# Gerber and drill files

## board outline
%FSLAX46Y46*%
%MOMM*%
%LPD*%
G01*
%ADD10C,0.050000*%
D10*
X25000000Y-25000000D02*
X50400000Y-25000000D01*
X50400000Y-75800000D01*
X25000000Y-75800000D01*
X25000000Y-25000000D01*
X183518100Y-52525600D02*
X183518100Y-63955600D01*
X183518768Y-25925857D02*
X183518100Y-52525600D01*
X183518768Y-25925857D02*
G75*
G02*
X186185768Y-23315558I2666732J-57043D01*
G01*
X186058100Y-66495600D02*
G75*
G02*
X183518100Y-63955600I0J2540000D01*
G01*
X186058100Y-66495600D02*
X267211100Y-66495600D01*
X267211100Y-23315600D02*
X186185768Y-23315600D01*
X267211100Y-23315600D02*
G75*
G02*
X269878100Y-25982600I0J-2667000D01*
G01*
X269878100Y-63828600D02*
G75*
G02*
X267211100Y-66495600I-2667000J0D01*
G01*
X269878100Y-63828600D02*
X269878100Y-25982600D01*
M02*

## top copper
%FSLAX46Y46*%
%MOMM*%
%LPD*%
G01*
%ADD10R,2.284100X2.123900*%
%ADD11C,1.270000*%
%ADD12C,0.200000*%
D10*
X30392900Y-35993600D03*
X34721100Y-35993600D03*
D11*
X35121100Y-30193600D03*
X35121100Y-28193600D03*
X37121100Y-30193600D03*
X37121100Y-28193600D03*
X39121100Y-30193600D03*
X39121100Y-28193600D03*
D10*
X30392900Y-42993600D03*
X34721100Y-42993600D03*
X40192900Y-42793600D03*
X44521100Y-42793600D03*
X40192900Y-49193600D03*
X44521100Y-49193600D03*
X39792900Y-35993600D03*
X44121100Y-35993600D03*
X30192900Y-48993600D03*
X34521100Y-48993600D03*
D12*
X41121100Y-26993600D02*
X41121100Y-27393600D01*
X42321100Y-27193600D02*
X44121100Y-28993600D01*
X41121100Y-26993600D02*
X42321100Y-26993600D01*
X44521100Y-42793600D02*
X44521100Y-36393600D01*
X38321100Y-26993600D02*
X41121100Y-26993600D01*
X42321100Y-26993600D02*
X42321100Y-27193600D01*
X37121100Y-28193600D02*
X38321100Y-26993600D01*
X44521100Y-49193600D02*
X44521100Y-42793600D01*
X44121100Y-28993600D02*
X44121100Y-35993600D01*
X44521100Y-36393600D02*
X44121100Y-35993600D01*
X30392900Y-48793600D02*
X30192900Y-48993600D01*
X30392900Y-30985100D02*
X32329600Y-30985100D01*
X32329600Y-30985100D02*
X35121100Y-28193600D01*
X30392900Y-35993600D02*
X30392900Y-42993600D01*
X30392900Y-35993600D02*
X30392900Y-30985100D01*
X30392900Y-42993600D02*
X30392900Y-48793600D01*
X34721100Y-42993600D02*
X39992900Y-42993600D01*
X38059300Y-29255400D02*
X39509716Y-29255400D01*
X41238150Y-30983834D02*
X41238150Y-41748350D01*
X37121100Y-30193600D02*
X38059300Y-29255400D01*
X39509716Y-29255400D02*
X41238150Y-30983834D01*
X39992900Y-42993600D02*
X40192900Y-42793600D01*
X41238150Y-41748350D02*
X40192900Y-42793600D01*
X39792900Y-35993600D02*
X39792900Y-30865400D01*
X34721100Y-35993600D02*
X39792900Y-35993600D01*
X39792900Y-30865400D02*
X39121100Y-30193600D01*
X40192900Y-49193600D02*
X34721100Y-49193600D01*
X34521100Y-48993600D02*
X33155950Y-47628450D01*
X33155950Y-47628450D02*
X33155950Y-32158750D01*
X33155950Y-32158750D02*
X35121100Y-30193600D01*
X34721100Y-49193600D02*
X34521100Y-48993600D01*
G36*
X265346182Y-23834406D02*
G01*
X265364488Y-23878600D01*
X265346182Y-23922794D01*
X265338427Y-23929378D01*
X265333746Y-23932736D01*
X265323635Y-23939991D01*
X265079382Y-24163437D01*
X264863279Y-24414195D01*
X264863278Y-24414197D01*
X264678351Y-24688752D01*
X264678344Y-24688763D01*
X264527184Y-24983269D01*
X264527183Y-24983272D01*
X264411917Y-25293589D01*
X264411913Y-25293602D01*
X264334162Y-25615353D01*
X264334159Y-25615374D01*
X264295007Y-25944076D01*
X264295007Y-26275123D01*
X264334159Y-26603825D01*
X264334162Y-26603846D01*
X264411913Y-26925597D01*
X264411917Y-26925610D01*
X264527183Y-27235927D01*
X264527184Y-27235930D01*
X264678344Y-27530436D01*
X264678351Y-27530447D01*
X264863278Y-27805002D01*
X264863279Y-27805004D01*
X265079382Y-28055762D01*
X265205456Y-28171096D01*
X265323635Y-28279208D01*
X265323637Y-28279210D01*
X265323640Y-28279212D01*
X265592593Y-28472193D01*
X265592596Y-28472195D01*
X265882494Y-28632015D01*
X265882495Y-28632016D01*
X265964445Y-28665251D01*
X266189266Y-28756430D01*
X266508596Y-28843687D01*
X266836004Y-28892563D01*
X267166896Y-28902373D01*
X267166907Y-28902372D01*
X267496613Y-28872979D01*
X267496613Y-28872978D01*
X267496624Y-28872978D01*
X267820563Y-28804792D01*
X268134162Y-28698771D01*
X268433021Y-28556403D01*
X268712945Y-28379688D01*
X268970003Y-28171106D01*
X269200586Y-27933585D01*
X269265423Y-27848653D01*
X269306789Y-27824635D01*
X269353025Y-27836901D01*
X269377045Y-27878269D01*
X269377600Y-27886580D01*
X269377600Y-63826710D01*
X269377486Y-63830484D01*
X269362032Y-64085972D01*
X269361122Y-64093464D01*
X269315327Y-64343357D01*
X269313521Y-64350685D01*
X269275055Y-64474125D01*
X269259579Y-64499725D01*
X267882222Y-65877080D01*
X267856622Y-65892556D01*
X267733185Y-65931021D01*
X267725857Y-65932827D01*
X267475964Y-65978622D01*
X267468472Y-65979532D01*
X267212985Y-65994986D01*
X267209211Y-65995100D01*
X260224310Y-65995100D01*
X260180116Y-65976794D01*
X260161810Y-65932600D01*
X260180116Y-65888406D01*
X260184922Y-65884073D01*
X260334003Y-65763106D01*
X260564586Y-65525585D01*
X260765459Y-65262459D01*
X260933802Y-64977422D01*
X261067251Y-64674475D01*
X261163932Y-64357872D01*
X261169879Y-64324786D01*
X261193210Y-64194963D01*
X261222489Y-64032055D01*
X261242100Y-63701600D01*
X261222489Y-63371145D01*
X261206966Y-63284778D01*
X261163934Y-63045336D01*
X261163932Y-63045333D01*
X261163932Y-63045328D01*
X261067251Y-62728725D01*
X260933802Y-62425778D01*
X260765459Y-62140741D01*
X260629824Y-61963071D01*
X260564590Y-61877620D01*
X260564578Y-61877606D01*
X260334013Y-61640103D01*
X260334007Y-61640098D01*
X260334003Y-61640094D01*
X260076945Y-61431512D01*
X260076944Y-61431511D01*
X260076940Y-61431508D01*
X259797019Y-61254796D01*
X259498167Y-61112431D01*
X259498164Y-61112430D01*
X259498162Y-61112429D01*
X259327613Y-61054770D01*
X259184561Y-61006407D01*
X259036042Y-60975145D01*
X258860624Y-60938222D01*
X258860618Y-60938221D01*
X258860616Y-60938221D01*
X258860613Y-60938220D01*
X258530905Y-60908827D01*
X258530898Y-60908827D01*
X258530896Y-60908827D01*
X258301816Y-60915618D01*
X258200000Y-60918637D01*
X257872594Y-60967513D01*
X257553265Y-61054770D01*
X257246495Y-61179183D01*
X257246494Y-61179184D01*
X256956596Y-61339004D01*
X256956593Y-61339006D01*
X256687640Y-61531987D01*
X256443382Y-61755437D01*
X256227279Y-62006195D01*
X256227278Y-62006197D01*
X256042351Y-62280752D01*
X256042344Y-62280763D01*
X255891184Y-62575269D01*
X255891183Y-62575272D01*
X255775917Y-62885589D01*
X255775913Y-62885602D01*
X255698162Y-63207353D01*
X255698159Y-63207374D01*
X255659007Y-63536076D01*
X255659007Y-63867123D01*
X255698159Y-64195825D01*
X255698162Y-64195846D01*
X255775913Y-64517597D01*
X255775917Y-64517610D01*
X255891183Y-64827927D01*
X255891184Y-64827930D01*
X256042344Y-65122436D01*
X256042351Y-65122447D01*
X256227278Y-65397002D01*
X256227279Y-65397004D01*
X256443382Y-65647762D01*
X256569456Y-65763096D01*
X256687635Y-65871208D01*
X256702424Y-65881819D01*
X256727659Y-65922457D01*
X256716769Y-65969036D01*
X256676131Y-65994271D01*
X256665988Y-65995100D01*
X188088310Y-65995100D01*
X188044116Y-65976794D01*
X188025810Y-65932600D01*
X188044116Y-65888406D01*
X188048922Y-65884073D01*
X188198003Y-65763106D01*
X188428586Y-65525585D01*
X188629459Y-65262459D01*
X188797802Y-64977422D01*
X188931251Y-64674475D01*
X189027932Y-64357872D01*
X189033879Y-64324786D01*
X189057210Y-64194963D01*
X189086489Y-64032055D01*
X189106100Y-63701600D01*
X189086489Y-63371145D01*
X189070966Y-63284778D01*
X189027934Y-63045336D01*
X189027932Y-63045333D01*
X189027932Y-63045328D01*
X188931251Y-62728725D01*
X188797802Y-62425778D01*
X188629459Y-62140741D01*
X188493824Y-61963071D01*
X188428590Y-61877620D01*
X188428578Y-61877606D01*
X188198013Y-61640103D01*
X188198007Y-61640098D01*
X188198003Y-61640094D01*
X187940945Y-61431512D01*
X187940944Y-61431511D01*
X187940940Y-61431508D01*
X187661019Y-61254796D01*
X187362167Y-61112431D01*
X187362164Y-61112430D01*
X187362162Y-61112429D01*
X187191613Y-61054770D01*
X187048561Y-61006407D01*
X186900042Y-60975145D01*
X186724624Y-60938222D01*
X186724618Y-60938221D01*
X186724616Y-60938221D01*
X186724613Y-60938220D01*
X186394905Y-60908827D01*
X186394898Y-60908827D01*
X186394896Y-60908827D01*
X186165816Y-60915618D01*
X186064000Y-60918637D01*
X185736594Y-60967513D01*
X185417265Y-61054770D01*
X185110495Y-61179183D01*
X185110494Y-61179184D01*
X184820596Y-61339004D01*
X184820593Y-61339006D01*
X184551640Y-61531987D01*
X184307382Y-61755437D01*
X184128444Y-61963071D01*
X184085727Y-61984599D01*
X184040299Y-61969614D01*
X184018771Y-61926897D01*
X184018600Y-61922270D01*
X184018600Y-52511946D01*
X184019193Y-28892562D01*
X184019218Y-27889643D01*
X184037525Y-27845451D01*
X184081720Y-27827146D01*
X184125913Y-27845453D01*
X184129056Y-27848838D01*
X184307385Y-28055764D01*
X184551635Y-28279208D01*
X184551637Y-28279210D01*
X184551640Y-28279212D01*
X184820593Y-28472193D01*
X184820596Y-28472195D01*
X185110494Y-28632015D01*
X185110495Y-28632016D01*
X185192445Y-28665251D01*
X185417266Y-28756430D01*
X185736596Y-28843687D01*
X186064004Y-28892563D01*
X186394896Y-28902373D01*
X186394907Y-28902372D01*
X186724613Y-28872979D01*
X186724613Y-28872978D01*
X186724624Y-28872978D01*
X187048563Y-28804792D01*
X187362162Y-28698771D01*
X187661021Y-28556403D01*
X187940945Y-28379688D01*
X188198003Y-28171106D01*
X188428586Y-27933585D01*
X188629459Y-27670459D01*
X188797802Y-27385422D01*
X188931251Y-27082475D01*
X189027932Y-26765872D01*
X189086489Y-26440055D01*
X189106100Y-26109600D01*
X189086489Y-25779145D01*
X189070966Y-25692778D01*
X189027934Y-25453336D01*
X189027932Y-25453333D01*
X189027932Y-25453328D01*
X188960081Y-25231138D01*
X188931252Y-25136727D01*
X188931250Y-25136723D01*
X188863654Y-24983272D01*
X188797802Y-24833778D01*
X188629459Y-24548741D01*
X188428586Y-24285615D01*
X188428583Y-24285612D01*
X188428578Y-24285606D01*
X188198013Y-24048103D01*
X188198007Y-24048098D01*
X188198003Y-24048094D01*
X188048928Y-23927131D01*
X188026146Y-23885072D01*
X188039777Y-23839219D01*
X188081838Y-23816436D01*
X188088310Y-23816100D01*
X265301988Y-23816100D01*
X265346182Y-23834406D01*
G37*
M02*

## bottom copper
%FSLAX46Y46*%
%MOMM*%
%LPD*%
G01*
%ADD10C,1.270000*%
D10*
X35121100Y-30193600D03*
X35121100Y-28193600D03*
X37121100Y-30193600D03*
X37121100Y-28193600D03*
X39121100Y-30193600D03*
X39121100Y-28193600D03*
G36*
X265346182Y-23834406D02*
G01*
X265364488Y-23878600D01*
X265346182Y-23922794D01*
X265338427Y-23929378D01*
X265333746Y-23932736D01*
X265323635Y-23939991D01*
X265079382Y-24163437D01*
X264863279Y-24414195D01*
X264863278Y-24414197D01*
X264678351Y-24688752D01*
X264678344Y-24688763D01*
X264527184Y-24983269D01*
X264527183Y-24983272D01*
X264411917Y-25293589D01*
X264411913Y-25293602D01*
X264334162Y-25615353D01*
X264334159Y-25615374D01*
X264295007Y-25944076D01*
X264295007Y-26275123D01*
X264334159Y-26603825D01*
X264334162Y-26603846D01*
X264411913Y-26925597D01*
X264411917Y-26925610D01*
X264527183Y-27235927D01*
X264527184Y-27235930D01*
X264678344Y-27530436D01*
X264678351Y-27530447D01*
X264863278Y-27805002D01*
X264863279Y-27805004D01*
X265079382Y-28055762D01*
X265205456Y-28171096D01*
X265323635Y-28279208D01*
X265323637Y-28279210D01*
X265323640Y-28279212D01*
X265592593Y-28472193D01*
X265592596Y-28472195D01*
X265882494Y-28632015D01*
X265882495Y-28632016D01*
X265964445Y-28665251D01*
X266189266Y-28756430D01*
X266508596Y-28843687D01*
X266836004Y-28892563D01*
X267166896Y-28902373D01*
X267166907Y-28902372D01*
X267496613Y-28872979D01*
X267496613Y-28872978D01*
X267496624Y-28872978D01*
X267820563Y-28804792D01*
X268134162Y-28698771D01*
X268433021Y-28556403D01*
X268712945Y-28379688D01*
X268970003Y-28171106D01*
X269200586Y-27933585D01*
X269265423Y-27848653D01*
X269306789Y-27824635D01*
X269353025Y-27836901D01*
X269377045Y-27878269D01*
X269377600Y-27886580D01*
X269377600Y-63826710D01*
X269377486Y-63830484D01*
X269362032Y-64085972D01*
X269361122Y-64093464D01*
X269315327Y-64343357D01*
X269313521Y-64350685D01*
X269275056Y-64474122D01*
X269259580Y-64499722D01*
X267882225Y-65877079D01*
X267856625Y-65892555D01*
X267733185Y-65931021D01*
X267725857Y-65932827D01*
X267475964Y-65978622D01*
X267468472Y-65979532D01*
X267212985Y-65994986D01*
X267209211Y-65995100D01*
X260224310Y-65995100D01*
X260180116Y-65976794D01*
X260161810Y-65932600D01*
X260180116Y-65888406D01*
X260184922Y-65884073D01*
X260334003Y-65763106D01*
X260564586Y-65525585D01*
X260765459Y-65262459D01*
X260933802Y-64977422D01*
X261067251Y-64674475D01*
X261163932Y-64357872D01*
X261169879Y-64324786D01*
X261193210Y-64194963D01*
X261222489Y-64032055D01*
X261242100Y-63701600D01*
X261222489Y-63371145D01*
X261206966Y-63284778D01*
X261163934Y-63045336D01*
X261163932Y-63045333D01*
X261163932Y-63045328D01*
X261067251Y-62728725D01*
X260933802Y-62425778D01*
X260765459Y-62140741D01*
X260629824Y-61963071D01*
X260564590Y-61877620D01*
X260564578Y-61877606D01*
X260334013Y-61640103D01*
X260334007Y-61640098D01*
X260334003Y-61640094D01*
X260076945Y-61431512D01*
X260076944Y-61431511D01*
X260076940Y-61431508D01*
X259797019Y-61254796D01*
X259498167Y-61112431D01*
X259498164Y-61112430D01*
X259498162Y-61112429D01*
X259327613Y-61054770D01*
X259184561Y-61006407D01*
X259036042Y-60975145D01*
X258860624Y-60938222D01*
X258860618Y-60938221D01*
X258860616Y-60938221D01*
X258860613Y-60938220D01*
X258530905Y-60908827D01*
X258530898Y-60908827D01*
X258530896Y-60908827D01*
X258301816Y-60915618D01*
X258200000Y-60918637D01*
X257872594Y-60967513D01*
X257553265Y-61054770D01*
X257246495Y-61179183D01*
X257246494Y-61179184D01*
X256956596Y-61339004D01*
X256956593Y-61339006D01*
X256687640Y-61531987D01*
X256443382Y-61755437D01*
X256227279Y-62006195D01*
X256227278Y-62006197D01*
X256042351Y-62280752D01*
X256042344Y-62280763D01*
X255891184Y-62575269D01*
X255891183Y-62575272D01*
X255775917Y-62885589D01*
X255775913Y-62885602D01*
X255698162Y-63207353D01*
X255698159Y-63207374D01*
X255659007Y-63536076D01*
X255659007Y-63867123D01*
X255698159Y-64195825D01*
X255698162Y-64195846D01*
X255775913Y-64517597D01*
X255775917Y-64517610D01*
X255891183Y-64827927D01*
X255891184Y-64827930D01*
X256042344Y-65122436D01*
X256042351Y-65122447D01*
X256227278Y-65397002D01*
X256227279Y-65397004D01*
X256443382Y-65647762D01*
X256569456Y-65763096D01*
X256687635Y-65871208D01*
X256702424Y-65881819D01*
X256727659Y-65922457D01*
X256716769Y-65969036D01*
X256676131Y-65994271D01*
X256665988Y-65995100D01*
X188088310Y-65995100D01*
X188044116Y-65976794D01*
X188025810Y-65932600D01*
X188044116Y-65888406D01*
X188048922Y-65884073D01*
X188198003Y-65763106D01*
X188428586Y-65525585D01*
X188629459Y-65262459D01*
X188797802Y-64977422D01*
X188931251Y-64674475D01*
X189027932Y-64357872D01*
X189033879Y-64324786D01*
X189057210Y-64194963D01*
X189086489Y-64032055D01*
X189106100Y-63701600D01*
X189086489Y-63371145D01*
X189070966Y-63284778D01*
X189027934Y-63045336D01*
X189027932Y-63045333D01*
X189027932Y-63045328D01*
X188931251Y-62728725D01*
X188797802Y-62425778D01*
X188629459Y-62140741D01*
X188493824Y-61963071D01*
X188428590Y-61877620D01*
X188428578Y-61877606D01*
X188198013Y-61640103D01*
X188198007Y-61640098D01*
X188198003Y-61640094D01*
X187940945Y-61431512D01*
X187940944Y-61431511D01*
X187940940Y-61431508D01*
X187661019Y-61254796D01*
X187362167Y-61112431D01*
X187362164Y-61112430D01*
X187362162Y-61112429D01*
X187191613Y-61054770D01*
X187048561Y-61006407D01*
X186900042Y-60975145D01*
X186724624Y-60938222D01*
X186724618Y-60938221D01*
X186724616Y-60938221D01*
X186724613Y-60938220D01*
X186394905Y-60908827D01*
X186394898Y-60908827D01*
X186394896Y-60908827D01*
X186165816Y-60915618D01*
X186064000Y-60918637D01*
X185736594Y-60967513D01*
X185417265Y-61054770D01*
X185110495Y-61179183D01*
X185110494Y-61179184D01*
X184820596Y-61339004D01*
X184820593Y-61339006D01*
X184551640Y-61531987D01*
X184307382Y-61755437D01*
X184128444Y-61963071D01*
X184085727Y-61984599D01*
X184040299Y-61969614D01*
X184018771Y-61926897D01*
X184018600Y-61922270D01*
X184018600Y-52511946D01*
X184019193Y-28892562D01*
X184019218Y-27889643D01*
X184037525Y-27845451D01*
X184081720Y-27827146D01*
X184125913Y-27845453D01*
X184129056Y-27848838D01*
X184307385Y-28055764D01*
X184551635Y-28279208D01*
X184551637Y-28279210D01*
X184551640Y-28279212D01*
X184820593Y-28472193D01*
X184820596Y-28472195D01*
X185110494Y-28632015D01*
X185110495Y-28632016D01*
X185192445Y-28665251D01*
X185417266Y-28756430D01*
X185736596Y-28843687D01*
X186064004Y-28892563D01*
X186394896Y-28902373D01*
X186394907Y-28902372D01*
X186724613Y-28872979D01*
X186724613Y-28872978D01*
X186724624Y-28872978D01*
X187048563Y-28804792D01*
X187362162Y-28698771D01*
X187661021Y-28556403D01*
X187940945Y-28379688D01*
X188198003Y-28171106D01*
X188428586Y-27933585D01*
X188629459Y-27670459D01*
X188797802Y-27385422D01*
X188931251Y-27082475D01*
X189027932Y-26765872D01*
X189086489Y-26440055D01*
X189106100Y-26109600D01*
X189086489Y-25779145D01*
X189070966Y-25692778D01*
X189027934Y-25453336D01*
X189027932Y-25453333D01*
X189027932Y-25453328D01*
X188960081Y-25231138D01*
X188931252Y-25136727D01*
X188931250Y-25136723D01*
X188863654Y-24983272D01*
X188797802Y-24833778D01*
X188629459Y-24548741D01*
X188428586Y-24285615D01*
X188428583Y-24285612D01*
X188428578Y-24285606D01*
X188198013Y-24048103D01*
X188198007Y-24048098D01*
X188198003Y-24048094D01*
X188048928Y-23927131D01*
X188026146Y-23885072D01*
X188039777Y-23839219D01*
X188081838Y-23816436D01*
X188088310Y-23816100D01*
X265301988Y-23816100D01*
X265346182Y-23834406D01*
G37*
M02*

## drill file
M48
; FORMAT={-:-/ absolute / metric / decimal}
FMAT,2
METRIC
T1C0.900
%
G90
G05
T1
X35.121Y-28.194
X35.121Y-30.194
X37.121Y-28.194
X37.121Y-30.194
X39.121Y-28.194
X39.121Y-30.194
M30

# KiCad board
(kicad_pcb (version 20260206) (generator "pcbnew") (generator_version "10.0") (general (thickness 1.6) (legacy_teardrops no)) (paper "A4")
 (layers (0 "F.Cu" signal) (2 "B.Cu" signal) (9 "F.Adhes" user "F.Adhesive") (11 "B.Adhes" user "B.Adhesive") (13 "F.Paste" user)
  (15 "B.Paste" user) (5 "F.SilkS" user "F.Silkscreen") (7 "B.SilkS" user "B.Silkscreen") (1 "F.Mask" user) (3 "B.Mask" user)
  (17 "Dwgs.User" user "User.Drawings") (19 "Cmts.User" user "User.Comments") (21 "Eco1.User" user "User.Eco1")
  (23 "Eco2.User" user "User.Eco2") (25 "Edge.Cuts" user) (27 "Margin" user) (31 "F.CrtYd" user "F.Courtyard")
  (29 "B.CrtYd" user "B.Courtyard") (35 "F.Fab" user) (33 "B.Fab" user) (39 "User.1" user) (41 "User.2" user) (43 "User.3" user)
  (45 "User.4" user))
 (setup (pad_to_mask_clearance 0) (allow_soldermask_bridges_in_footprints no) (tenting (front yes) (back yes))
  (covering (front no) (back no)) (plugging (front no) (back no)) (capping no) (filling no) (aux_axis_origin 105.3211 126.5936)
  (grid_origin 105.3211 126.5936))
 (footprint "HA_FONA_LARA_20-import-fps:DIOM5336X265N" (layer "F.Cu") (at 32.557 35.9936)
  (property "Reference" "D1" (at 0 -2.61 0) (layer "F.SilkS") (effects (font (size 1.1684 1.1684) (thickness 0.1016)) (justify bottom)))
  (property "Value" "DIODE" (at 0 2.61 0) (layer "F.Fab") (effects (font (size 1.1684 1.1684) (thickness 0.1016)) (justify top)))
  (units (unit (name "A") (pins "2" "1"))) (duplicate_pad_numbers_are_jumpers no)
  (pad "1" smd rect (at -2.1641 0) (size 2.2841 2.1239) (layers "F.Cu" "F.Mask" "F.Paste") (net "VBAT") (solder_mask_margin 0.0508)
   (solder_paste_margin 0) (thermal_bridge_angle 0))
  (pad "2" smd rect (at 2.1641 0) (size 2.2841 2.1239) (layers "F.Cu" "F.Mask" "F.Paste") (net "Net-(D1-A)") (solder_mask_margin 0.0508)
   (solder_paste_margin 0) (thermal_bridge_angle 0)))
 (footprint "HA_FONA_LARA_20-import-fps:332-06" (layer "F.Cu") (at 37.1211 29.1936)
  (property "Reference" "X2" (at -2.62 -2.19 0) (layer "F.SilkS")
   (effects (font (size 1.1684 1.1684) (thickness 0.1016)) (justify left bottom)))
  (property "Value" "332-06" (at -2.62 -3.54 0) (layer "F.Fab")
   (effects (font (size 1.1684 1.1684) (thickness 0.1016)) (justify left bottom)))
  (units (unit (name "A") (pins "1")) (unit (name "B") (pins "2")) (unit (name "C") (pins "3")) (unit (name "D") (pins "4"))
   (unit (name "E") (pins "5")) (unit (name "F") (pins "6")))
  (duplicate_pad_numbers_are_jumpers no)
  (pad "1" thru_hole circle (at -2 1) (size 1.27 1.27) (drill 0.9) (layers "*.Cu" "*.Mask") (remove_unused_layers no) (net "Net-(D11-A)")
   (solder_mask_margin 0.0508) (thermal_bridge_angle 0))
  (pad "2" thru_hole circle (at -2 -1) (size 1.27 1.27) (drill 0.9) (layers "*.Cu" "*.Mask") (remove_unused_layers no) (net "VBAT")
   (solder_mask_margin 0.0508) (thermal_bridge_angle 0))
  (pad "3" thru_hole circle (at 0 1) (size 1.27 1.27) (drill 0.9) (layers "*.Cu" "*.Mask") (remove_unused_layers no) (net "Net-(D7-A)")
   (solder_mask_margin 0.0508) (thermal_bridge_angle 0))
  (pad "4" thru_hole circle (at 0 -1) (size 1.27 1.27) (drill 0.9) (layers "*.Cu" "*.Mask") (remove_unused_layers no) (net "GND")
   (solder_mask_margin 0.0508) (thermal_bridge_angle 0))
  (pad "5" thru_hole circle (at 2 1) (size 1.27 1.27) (drill 0.9) (layers "*.Cu" "*.Mask") (remove_unused_layers no) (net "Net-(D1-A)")
   (solder_mask_margin 0.0508) (thermal_bridge_angle 0))
  (pad "6" thru_hole circle (at 2 -1) (size 1.27 1.27) (drill 0.9) (layers "*.Cu" "*.Mask") (remove_unused_layers no)
   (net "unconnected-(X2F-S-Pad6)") (solder_mask_margin 0.0508) (thermal_bridge_angle 0)))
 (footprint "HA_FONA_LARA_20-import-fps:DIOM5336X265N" (layer "F.Cu") (at 32.557 42.9936)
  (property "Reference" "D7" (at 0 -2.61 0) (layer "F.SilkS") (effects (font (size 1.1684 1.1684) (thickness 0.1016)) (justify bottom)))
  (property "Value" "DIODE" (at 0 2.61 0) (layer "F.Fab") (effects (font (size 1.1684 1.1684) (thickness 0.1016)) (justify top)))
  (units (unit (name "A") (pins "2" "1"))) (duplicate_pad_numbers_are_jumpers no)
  (pad "1" smd rect (at -2.1641 0) (size 2.2841 2.1239) (layers "F.Cu" "F.Mask" "F.Paste") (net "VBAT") (solder_mask_margin 0.0508)
   (solder_paste_margin 0) (thermal_bridge_angle 0))
  (pad "2" smd rect (at 2.1641 0) (size 2.2841 2.1239) (layers "F.Cu" "F.Mask" "F.Paste") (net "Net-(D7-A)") (solder_mask_margin 0.0508)
   (solder_paste_margin 0) (thermal_bridge_angle 0)))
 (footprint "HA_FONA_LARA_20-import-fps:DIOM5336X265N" (layer "F.Cu") (at 42.357 42.7936)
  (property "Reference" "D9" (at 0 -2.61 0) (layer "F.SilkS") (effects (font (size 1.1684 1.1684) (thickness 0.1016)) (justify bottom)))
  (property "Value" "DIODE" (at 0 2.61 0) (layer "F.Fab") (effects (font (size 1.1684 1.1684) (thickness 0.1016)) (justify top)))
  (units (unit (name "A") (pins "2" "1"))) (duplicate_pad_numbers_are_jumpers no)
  (pad "1" smd rect (at -2.1641 0) (size 2.2841 2.1239) (layers "F.Cu" "F.Mask" "F.Paste") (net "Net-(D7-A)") (solder_mask_margin 0.0508)
   (solder_paste_margin 0) (thermal_bridge_angle 0))
  (pad "2" smd rect (at 2.1641 0) (size 2.2841 2.1239) (layers "F.Cu" "F.Mask" "F.Paste") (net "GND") (solder_mask_margin 0.0508)
   (solder_paste_margin 0) (thermal_bridge_angle 0)))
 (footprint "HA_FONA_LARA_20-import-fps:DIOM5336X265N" (layer "F.Cu") (at 42.357 49.1936)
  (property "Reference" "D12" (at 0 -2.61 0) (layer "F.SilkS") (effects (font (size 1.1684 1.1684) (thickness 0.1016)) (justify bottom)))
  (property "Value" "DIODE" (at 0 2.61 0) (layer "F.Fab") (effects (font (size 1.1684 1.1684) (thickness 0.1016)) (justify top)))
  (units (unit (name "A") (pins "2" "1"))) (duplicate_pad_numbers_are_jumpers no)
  (pad "1" smd rect (at -2.1641 0) (size 2.2841 2.1239) (layers "F.Cu" "F.Mask" "F.Paste") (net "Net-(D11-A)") (solder_mask_margin 0.0508)
   (solder_paste_margin 0) (thermal_bridge_angle 0))
  (pad "2" smd rect (at 2.1641 0) (size 2.2841 2.1239) (layers "F.Cu" "F.Mask" "F.Paste") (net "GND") (solder_mask_margin 0.0508)
   (solder_paste_margin 0) (thermal_bridge_angle 0)))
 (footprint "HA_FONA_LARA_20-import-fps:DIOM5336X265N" (layer "F.Cu") (at 41.957 35.9936)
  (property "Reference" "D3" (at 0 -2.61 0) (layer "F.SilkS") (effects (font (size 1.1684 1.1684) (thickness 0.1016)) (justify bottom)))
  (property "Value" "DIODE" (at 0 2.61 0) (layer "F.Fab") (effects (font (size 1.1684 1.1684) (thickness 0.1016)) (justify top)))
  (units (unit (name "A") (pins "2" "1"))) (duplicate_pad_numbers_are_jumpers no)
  (pad "1" smd rect (at -2.1641 0) (size 2.2841 2.1239) (layers "F.Cu" "F.Mask" "F.Paste") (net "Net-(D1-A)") (solder_mask_margin 0.0508)
   (solder_paste_margin 0) (thermal_bridge_angle 0))
  (pad "2" smd rect (at 2.1641 0) (size 2.2841 2.1239) (layers "F.Cu" "F.Mask" "F.Paste") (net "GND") (solder_mask_margin 0.0508)
   (solder_paste_margin 0) (thermal_bridge_angle 0)))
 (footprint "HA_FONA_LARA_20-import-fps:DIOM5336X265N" (layer "F.Cu") (at 32.357 48.9936)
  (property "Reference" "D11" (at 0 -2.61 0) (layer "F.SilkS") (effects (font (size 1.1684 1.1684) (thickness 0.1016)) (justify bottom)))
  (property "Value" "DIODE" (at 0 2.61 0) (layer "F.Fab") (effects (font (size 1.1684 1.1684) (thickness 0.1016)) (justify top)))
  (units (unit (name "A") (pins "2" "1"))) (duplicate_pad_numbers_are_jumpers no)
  (pad "1" smd rect (at -2.1641 0) (size 2.2841 2.1239) (layers "F.Cu" "F.Mask" "F.Paste") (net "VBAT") (solder_mask_margin 0.0508)
   (solder_paste_margin 0) (thermal_bridge_angle 0))
  (pad "2" smd rect (at 2.1641 0) (size 2.2841 2.1239) (layers "F.Cu" "F.Mask" "F.Paste") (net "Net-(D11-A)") (solder_mask_margin 0.0508)
   (solder_paste_margin 0) (thermal_bridge_angle 0)))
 (gr_rect (start 25 25) (end 50.4 75.8) (stroke (width 0.05) (type solid)) (fill no) (layer "Edge.Cuts"))
 (gr_line (start 183.5181 52.5256) (end 183.5181 63.9556) (stroke (width 0.05) (type solid)) (layer "Edge.Cuts"))
 (gr_line (start 183.518768 25.925857) (end 183.5181 52.5256) (stroke (width 0.05) (type solid)) (layer "Edge.Cuts"))
 (gr_arc (start 183.518768 25.925857) (mid 184.31978 24.076665) (end 186.185768 23.3156) (stroke (width 0.05) (type solid))
  (layer "Edge.Cuts"))
 (gr_arc (start 186.0581 66.4956) (mid 184.262049 65.751651) (end 183.5181 63.9556) (stroke (width 0.05) (type solid)) (layer "Edge.Cuts"))
 (gr_line (start 186.0581 66.4956) (end 267.2111 66.4956) (stroke (width 0.05) (type solid)) (layer "Edge.Cuts"))
 (gr_line (start 267.2111 23.3156) (end 186.185768 23.3156) (stroke (width 0.05) (type solid)) (layer "Edge.Cuts"))
 (gr_arc (start 267.2111 23.3156) (mid 269.096954 24.096746) (end 269.8781 25.9826) (stroke (width 0.05) (type solid)) (layer "Edge.Cuts"))
 (gr_arc (start 269.8781 63.8286) (mid 269.096954 65.714454) (end 267.2111 66.4956) (stroke (width 0.05) (type solid)) (layer "Edge.Cuts"))
 (gr_line (start 269.8781 63.8286) (end 269.8781 25.9826) (stroke (width 0.05) (type solid)) (layer "Edge.Cuts"))
 (segment (start 41.1211 26.9936) (end 41.1211 27.3936) (width 0.2) (layer "F.Cu") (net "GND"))
 (segment (start 42.3211 27.1936) (end 44.1211 28.9936) (width 0.2) (layer "F.Cu") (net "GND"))
 (segment (start 41.1211 26.9936) (end 42.3211 26.9936) (width 0.2) (layer "F.Cu") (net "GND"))
 (segment (start 44.5211 42.7936) (end 44.5211 36.3936) (width 0.2) (layer "F.Cu") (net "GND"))
 (segment (start 38.3211 26.9936) (end 41.1211 26.9936) (width 0.2) (layer "F.Cu") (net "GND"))
 (segment (start 42.3211 26.9936) (end 42.3211 27.1936) (width 0.2) (layer "F.Cu") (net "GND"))
 (segment (start 37.1211 28.1936) (end 38.3211 26.9936) (width 0.2) (layer "F.Cu") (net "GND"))
 (segment (start 44.5211 49.1936) (end 44.5211 42.7936) (width 0.2) (layer "F.Cu") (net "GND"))
 (segment (start 44.1211 28.9936) (end 44.1211 35.9936) (width 0.2) (layer "F.Cu") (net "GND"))
 (segment (start 44.5211 36.3936) (end 44.1211 35.9936) (width 0.2) (layer "F.Cu") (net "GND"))
 (segment (start 30.3929 48.7936) (end 30.1929 48.9936) (width 0.2) (layer "F.Cu") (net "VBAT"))
 (segment (start 30.3929 30.9851) (end 32.3296 30.9851) (width 0.2) (layer "F.Cu") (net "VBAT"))
 (segment (start 32.3296 30.9851) (end 35.1211 28.1936) (width 0.2) (layer "F.Cu") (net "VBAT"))
 (segment (start 30.3929 35.9936) (end 30.3929 42.9936) (width 0.2) (layer "F.Cu") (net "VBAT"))
 (segment (start 30.3929 35.9936) (end 30.3929 30.9851) (width 0.2) (layer "F.Cu") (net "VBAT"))
 (segment (start 30.3929 42.9936) (end 30.3929 48.7936) (width 0.2) (layer "F.Cu") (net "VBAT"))
 (segment (start 34.7211 42.9936) (end 39.9929 42.9936) (width 0.2) (layer "F.Cu") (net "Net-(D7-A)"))
 (segment (start 38.0593 29.2554) (end 39.509716 29.2554) (width 0.2) (layer "F.Cu") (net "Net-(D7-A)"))
 (segment (start 41.23815 30.983834) (end 41.23815 41.74835) (width 0.2) (layer "F.Cu") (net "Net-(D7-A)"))
 (segment (start 37.1211 30.1936) (end 38.0593 29.2554) (width 0.2) (layer "F.Cu") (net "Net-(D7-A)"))
 (segment (start 39.509716 29.2554) (end 41.23815 30.983834) (width 0.2) (layer "F.Cu") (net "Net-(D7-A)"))
 (segment (start 39.9929 42.9936) (end 40.1929 42.7936) (width 0.2) (layer "F.Cu") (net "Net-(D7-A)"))
 (segment (start 41.23815 41.74835) (end 40.1929 42.7936) (width 0.2) (layer "F.Cu") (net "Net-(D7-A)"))
 (segment (start 39.7929 35.9936) (end 39.7929 30.8654) (width 0.2) (layer "F.Cu") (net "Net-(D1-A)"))
 (segment (start 34.7211 35.9936) (end 39.7929 35.9936) (width 0.2) (layer "F.Cu") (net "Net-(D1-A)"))
 (segment (start 39.7929 30.8654) (end 39.1211 30.1936) (width 0.2) (layer "F.Cu") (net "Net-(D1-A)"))
 (segment (start 40.1929 49.1936) (end 34.7211 49.1936) (width 0.2) (layer "F.Cu") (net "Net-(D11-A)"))
 (segment (start 34.5211 48.9936) (end 33.15595 47.62845) (width 0.2) (layer "F.Cu") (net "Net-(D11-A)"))
 (segment (start 33.15595 47.62845) (end 33.15595 32.15875) (width 0.2) (layer "F.Cu") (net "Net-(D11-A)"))
 (segment (start 33.15595 32.15875) (end 35.1211 30.1936) (width 0.2) (layer "F.Cu") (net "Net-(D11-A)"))
 (segment (start 34.7211 49.1936) (end 34.5211 48.9936) (width 0.2) (layer "F.Cu") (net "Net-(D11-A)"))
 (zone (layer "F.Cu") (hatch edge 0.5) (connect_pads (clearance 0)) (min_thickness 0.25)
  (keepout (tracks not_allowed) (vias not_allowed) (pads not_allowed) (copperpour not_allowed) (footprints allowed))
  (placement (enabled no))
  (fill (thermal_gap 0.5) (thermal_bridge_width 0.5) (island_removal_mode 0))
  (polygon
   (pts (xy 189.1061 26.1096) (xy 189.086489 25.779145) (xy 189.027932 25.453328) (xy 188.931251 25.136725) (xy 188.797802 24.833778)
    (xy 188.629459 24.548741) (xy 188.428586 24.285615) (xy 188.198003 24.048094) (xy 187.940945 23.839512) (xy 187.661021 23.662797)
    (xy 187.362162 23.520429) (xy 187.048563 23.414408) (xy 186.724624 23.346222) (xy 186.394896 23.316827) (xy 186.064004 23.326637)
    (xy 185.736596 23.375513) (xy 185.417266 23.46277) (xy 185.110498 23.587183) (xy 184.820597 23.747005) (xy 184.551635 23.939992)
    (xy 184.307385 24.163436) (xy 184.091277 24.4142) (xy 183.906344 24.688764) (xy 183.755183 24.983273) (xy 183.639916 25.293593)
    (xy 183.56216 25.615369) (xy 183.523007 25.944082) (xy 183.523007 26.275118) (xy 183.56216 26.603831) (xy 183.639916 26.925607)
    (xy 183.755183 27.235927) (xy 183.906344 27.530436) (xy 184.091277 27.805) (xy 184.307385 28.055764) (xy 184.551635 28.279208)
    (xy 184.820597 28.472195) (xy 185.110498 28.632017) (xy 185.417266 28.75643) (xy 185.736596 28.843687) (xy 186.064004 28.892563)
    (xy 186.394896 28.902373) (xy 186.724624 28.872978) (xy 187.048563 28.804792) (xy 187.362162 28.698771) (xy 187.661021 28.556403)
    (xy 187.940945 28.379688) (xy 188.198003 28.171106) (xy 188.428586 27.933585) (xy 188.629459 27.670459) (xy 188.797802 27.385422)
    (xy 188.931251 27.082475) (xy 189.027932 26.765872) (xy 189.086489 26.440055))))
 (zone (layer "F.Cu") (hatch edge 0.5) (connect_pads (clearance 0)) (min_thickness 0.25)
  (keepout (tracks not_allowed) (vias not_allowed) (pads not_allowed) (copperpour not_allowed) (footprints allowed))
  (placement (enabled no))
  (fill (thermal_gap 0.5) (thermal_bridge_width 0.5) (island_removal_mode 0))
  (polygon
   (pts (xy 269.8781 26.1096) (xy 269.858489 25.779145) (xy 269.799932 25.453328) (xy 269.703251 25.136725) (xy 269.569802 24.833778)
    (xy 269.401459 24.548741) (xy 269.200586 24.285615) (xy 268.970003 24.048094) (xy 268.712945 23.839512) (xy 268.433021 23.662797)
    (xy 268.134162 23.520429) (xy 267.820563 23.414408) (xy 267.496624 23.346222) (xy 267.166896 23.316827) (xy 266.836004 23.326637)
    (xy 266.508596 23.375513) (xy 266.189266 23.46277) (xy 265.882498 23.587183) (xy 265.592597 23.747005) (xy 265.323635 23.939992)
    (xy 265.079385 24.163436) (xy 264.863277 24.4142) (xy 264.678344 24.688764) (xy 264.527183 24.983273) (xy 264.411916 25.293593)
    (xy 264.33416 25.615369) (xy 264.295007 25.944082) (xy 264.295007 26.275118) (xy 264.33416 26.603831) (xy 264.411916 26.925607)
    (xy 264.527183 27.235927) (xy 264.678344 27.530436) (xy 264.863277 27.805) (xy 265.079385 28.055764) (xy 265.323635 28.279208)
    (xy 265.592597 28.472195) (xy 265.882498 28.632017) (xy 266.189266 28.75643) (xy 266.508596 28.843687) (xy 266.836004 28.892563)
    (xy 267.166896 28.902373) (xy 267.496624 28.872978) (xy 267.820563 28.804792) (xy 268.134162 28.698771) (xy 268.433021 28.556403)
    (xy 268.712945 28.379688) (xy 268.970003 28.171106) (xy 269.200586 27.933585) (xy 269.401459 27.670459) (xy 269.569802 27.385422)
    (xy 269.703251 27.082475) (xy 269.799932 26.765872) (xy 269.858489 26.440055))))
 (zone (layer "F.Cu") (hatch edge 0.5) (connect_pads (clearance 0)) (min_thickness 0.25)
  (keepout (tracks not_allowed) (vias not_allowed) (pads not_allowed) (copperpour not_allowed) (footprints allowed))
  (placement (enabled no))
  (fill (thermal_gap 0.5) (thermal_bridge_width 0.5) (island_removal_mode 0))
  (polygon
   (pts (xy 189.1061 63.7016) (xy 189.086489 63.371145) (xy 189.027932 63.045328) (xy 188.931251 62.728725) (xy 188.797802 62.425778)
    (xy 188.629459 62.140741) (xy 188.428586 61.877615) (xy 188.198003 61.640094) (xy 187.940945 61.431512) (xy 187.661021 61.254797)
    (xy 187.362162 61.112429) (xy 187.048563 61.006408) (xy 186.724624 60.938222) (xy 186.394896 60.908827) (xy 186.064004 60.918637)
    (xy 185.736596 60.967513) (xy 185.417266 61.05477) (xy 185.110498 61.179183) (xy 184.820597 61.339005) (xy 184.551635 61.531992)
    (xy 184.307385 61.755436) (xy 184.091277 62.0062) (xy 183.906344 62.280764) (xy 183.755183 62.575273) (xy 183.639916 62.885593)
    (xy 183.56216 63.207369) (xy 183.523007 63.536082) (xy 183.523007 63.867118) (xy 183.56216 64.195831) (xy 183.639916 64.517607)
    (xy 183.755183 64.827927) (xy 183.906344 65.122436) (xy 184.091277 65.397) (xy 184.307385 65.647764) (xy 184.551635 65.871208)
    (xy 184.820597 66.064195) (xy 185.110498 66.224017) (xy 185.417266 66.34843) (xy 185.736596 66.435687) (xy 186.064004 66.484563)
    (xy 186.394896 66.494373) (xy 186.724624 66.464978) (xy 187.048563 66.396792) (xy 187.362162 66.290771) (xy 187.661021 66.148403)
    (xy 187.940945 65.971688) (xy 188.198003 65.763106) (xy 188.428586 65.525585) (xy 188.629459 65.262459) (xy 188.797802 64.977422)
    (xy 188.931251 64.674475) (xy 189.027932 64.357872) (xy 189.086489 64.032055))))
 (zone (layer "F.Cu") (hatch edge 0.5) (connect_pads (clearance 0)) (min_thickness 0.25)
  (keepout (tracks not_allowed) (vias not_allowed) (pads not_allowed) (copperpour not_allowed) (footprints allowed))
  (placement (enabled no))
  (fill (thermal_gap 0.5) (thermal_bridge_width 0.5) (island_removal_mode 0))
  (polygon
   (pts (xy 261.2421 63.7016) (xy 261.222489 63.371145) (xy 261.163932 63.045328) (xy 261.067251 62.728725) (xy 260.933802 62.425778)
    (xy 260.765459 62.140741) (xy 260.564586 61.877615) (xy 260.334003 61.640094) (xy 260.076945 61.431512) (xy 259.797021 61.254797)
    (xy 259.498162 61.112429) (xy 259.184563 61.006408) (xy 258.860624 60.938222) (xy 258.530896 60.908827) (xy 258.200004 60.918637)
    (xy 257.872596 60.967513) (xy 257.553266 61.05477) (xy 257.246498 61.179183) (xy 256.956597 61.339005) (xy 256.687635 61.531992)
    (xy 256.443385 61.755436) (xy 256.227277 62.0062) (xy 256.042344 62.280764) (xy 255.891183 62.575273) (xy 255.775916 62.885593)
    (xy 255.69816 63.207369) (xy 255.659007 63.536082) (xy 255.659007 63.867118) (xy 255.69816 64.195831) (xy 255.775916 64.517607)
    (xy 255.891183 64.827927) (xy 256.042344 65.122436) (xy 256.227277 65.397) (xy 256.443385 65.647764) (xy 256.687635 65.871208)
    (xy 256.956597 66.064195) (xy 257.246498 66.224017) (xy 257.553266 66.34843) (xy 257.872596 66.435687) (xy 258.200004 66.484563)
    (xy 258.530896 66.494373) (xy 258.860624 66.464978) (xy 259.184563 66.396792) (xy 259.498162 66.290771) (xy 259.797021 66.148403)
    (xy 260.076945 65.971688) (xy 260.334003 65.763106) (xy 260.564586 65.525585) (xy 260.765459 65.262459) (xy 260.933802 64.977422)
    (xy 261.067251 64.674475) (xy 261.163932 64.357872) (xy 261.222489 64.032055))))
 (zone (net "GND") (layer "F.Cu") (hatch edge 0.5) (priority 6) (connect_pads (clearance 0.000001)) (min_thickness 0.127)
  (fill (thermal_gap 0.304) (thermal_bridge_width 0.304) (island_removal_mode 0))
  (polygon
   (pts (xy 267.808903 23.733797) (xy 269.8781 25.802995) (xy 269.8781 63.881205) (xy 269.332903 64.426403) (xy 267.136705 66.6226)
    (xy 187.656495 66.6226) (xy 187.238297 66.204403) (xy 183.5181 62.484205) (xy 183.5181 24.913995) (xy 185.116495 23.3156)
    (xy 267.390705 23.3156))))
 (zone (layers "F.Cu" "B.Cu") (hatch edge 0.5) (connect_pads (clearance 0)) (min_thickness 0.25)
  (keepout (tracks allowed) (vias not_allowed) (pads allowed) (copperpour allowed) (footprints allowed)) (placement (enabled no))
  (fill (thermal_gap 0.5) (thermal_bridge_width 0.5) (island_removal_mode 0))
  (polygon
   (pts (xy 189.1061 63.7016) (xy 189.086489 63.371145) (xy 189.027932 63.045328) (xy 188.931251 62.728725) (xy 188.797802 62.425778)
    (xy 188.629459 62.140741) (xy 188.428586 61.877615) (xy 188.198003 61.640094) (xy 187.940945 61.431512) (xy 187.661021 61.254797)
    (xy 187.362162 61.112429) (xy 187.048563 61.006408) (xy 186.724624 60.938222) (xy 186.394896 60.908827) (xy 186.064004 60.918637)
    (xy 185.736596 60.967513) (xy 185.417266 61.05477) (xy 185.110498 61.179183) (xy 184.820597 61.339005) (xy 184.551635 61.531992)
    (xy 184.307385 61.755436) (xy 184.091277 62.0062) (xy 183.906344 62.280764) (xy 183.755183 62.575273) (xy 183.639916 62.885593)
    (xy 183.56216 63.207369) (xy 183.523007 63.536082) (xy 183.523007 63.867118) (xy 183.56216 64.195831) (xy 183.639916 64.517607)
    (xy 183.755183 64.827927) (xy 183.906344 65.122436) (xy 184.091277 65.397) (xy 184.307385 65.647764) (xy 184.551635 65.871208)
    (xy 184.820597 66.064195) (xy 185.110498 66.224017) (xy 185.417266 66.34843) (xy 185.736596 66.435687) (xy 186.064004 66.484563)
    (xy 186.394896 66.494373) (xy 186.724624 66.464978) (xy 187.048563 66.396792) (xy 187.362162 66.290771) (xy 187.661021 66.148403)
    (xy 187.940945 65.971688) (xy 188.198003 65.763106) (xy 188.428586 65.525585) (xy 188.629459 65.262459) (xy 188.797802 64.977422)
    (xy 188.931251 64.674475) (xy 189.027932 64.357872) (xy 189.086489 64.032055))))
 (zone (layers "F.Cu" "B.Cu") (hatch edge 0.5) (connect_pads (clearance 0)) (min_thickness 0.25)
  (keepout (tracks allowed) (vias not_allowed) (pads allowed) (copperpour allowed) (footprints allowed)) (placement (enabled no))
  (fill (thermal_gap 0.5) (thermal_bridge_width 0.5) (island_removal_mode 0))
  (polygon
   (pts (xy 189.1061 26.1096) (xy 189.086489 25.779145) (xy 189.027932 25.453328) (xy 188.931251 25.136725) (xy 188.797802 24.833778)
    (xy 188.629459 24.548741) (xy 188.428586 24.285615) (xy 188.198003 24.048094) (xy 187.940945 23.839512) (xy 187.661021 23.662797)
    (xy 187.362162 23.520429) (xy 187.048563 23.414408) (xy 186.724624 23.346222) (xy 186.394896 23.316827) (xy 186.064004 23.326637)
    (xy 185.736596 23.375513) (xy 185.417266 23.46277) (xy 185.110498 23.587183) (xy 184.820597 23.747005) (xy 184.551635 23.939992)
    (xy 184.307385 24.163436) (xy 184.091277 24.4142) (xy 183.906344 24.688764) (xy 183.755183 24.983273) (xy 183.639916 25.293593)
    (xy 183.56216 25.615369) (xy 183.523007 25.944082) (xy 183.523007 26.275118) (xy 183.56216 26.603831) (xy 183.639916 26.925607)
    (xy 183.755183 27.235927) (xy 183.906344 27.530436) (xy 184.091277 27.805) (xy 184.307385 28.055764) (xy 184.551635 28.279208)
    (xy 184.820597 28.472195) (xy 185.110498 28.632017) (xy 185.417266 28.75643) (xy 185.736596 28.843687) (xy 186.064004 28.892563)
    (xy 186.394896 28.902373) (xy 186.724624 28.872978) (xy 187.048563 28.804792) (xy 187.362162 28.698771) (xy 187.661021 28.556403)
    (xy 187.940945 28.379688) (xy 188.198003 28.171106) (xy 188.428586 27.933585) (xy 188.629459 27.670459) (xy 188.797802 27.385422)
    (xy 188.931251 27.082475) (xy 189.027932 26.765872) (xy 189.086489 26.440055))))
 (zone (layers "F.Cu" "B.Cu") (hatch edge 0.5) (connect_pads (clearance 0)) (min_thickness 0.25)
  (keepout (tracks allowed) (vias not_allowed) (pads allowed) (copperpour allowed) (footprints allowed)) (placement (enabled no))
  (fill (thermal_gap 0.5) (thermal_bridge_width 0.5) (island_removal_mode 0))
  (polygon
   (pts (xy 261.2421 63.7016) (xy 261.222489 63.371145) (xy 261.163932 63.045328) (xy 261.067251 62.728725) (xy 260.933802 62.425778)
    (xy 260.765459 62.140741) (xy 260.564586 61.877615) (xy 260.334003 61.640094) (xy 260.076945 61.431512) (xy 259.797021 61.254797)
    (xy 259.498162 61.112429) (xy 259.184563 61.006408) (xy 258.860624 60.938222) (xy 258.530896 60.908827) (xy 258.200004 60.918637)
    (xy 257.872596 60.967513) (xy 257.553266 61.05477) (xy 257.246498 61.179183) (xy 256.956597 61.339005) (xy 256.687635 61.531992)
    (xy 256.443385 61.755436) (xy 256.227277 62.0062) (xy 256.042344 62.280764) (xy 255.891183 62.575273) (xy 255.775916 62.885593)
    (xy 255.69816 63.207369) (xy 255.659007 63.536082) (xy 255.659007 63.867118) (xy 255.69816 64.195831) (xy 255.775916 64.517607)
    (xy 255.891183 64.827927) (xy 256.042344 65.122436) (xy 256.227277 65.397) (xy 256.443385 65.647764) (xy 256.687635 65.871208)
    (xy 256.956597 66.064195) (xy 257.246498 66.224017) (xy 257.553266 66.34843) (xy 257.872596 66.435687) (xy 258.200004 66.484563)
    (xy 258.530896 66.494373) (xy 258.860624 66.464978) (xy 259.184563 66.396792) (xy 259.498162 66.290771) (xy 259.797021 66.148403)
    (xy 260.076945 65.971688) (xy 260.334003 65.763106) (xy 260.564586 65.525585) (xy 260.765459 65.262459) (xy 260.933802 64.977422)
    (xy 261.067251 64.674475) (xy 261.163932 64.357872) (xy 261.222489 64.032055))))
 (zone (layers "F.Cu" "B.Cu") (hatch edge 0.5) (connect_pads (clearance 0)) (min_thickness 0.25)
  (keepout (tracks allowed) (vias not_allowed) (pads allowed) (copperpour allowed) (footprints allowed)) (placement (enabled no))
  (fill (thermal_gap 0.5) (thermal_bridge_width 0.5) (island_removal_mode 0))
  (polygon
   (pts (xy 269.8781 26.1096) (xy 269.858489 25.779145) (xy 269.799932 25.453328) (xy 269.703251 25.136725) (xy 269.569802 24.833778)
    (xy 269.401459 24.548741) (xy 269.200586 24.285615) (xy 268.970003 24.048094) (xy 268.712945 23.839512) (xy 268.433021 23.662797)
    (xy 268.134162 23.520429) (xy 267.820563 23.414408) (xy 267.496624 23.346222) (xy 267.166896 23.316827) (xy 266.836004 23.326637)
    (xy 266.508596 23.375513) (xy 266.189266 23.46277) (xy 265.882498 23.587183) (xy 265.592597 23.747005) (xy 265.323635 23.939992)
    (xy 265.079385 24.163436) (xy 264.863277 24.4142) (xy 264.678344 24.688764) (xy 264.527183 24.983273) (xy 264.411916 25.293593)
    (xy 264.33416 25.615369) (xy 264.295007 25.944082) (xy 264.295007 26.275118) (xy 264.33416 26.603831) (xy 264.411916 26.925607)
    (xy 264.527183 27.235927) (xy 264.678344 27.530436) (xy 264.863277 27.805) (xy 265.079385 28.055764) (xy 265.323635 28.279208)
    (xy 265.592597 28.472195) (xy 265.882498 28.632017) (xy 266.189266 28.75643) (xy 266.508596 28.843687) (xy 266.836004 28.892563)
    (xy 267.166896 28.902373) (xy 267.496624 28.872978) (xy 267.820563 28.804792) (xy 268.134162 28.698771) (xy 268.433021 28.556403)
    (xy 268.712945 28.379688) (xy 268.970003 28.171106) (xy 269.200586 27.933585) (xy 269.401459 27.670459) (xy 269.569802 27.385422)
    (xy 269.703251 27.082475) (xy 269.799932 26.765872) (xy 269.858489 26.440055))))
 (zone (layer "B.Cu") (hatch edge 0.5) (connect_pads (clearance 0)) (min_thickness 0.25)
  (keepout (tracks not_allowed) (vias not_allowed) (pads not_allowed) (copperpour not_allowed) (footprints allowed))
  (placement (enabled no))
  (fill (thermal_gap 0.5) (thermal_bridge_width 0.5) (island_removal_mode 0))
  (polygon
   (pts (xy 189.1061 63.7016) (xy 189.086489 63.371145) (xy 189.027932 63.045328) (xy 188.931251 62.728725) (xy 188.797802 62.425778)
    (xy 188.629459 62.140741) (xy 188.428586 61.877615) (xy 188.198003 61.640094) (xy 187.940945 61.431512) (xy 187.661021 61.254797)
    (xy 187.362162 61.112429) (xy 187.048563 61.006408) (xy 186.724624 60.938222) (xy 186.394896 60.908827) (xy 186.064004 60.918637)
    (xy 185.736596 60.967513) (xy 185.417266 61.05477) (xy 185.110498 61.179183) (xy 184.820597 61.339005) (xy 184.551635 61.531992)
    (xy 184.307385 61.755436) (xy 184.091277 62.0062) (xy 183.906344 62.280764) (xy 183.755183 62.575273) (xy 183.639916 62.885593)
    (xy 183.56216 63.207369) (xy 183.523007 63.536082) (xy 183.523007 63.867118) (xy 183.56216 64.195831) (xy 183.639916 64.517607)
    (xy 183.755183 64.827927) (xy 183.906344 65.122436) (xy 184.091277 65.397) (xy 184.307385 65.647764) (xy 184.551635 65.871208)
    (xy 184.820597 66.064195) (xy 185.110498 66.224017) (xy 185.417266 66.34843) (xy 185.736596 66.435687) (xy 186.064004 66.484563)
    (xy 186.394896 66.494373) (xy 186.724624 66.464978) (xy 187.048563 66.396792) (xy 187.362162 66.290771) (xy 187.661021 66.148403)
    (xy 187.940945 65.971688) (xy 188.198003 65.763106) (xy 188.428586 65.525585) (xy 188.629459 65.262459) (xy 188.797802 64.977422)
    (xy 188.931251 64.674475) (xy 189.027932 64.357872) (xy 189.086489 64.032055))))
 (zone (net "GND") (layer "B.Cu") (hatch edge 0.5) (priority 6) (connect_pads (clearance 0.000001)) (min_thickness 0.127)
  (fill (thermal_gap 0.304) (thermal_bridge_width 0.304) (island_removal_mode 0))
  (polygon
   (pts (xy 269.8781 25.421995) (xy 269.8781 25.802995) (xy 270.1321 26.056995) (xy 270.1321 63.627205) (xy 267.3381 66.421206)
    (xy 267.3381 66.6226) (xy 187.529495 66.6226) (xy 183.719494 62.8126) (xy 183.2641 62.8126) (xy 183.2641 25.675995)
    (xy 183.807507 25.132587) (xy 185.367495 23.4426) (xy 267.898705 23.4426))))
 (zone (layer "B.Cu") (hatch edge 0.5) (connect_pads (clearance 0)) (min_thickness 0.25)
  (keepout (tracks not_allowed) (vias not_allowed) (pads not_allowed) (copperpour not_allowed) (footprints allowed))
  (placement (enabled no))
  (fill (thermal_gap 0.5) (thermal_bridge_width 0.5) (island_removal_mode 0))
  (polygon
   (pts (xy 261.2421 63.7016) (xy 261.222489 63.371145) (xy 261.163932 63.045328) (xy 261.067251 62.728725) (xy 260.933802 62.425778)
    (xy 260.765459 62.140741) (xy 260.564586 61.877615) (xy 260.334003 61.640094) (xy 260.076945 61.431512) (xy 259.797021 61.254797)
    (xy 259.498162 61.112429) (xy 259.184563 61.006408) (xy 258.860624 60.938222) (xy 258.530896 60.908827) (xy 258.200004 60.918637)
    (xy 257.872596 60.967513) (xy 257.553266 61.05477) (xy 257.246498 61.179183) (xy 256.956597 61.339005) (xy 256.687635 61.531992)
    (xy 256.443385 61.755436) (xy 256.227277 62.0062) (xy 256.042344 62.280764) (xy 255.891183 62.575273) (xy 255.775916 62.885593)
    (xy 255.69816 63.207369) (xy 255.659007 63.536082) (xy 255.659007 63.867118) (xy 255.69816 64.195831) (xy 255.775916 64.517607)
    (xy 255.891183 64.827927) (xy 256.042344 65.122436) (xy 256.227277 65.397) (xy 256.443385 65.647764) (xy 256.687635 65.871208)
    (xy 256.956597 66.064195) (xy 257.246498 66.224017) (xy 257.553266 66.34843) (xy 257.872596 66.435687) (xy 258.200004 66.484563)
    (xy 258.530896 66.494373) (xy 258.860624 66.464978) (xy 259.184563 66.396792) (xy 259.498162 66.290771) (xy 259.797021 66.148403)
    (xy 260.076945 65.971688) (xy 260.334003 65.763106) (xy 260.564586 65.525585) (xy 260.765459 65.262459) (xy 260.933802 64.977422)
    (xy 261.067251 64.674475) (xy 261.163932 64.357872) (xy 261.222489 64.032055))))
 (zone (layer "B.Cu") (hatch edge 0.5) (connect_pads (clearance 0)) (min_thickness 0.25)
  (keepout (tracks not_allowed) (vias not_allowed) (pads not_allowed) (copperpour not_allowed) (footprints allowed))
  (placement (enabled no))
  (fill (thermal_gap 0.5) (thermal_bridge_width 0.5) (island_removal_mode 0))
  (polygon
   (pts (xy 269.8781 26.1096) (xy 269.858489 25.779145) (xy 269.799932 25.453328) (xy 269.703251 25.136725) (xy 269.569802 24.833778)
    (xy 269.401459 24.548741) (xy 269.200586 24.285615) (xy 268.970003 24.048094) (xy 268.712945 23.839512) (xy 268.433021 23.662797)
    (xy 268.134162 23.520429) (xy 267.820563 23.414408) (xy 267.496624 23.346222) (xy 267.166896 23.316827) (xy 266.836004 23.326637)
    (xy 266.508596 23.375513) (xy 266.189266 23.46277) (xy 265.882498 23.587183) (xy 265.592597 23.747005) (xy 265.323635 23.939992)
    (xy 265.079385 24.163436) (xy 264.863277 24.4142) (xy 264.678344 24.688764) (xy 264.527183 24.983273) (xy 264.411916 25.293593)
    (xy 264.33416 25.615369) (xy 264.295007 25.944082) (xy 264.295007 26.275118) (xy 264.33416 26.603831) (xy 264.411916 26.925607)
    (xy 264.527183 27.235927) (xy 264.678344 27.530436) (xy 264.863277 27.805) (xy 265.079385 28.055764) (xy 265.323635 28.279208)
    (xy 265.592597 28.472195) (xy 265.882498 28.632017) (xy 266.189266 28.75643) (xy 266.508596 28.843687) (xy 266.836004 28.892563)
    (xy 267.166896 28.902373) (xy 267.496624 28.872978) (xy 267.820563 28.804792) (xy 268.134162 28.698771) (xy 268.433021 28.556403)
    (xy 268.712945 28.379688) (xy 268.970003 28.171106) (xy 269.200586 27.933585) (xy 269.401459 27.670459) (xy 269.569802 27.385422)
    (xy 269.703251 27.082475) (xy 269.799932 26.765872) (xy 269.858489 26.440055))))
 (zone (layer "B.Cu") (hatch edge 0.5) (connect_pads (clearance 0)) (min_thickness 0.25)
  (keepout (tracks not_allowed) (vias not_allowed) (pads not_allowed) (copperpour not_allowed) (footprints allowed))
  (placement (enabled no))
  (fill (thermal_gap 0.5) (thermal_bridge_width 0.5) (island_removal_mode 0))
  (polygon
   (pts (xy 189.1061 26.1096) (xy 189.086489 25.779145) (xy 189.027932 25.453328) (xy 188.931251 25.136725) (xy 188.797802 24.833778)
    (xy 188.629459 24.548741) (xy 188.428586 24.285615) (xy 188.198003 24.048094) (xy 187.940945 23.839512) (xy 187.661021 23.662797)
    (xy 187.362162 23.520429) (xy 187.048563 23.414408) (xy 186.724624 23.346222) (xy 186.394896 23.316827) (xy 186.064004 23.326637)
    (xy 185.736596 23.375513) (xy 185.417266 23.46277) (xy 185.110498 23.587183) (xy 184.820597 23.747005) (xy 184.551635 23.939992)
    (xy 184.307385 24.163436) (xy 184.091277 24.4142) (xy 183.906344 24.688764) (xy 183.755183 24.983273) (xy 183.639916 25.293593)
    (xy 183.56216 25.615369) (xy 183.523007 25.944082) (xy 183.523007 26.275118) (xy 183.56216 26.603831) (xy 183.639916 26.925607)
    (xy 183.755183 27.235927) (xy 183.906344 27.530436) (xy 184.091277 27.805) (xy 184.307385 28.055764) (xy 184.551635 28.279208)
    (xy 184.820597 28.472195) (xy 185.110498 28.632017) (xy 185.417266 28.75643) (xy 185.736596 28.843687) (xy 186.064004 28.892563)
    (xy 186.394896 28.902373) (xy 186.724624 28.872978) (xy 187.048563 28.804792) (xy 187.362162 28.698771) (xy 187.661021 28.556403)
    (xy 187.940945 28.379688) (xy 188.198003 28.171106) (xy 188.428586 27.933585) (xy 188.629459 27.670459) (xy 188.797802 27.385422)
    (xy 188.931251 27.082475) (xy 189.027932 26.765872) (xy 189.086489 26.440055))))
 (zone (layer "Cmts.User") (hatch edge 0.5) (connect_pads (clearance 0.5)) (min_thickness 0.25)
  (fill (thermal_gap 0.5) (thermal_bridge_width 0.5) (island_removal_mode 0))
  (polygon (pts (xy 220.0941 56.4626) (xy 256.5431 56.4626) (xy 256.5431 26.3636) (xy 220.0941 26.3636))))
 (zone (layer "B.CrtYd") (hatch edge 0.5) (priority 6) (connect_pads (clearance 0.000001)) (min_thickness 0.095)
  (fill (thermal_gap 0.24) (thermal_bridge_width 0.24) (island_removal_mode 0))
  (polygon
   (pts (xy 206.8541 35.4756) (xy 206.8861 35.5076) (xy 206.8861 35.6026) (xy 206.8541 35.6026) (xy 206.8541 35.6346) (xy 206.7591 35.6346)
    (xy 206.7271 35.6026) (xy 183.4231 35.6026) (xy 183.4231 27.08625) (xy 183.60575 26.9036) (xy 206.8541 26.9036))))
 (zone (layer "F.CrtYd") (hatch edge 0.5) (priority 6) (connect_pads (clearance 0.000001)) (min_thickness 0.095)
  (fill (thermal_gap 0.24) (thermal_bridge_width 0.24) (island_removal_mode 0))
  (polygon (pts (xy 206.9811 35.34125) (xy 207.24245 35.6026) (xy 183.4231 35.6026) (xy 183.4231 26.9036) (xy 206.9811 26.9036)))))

